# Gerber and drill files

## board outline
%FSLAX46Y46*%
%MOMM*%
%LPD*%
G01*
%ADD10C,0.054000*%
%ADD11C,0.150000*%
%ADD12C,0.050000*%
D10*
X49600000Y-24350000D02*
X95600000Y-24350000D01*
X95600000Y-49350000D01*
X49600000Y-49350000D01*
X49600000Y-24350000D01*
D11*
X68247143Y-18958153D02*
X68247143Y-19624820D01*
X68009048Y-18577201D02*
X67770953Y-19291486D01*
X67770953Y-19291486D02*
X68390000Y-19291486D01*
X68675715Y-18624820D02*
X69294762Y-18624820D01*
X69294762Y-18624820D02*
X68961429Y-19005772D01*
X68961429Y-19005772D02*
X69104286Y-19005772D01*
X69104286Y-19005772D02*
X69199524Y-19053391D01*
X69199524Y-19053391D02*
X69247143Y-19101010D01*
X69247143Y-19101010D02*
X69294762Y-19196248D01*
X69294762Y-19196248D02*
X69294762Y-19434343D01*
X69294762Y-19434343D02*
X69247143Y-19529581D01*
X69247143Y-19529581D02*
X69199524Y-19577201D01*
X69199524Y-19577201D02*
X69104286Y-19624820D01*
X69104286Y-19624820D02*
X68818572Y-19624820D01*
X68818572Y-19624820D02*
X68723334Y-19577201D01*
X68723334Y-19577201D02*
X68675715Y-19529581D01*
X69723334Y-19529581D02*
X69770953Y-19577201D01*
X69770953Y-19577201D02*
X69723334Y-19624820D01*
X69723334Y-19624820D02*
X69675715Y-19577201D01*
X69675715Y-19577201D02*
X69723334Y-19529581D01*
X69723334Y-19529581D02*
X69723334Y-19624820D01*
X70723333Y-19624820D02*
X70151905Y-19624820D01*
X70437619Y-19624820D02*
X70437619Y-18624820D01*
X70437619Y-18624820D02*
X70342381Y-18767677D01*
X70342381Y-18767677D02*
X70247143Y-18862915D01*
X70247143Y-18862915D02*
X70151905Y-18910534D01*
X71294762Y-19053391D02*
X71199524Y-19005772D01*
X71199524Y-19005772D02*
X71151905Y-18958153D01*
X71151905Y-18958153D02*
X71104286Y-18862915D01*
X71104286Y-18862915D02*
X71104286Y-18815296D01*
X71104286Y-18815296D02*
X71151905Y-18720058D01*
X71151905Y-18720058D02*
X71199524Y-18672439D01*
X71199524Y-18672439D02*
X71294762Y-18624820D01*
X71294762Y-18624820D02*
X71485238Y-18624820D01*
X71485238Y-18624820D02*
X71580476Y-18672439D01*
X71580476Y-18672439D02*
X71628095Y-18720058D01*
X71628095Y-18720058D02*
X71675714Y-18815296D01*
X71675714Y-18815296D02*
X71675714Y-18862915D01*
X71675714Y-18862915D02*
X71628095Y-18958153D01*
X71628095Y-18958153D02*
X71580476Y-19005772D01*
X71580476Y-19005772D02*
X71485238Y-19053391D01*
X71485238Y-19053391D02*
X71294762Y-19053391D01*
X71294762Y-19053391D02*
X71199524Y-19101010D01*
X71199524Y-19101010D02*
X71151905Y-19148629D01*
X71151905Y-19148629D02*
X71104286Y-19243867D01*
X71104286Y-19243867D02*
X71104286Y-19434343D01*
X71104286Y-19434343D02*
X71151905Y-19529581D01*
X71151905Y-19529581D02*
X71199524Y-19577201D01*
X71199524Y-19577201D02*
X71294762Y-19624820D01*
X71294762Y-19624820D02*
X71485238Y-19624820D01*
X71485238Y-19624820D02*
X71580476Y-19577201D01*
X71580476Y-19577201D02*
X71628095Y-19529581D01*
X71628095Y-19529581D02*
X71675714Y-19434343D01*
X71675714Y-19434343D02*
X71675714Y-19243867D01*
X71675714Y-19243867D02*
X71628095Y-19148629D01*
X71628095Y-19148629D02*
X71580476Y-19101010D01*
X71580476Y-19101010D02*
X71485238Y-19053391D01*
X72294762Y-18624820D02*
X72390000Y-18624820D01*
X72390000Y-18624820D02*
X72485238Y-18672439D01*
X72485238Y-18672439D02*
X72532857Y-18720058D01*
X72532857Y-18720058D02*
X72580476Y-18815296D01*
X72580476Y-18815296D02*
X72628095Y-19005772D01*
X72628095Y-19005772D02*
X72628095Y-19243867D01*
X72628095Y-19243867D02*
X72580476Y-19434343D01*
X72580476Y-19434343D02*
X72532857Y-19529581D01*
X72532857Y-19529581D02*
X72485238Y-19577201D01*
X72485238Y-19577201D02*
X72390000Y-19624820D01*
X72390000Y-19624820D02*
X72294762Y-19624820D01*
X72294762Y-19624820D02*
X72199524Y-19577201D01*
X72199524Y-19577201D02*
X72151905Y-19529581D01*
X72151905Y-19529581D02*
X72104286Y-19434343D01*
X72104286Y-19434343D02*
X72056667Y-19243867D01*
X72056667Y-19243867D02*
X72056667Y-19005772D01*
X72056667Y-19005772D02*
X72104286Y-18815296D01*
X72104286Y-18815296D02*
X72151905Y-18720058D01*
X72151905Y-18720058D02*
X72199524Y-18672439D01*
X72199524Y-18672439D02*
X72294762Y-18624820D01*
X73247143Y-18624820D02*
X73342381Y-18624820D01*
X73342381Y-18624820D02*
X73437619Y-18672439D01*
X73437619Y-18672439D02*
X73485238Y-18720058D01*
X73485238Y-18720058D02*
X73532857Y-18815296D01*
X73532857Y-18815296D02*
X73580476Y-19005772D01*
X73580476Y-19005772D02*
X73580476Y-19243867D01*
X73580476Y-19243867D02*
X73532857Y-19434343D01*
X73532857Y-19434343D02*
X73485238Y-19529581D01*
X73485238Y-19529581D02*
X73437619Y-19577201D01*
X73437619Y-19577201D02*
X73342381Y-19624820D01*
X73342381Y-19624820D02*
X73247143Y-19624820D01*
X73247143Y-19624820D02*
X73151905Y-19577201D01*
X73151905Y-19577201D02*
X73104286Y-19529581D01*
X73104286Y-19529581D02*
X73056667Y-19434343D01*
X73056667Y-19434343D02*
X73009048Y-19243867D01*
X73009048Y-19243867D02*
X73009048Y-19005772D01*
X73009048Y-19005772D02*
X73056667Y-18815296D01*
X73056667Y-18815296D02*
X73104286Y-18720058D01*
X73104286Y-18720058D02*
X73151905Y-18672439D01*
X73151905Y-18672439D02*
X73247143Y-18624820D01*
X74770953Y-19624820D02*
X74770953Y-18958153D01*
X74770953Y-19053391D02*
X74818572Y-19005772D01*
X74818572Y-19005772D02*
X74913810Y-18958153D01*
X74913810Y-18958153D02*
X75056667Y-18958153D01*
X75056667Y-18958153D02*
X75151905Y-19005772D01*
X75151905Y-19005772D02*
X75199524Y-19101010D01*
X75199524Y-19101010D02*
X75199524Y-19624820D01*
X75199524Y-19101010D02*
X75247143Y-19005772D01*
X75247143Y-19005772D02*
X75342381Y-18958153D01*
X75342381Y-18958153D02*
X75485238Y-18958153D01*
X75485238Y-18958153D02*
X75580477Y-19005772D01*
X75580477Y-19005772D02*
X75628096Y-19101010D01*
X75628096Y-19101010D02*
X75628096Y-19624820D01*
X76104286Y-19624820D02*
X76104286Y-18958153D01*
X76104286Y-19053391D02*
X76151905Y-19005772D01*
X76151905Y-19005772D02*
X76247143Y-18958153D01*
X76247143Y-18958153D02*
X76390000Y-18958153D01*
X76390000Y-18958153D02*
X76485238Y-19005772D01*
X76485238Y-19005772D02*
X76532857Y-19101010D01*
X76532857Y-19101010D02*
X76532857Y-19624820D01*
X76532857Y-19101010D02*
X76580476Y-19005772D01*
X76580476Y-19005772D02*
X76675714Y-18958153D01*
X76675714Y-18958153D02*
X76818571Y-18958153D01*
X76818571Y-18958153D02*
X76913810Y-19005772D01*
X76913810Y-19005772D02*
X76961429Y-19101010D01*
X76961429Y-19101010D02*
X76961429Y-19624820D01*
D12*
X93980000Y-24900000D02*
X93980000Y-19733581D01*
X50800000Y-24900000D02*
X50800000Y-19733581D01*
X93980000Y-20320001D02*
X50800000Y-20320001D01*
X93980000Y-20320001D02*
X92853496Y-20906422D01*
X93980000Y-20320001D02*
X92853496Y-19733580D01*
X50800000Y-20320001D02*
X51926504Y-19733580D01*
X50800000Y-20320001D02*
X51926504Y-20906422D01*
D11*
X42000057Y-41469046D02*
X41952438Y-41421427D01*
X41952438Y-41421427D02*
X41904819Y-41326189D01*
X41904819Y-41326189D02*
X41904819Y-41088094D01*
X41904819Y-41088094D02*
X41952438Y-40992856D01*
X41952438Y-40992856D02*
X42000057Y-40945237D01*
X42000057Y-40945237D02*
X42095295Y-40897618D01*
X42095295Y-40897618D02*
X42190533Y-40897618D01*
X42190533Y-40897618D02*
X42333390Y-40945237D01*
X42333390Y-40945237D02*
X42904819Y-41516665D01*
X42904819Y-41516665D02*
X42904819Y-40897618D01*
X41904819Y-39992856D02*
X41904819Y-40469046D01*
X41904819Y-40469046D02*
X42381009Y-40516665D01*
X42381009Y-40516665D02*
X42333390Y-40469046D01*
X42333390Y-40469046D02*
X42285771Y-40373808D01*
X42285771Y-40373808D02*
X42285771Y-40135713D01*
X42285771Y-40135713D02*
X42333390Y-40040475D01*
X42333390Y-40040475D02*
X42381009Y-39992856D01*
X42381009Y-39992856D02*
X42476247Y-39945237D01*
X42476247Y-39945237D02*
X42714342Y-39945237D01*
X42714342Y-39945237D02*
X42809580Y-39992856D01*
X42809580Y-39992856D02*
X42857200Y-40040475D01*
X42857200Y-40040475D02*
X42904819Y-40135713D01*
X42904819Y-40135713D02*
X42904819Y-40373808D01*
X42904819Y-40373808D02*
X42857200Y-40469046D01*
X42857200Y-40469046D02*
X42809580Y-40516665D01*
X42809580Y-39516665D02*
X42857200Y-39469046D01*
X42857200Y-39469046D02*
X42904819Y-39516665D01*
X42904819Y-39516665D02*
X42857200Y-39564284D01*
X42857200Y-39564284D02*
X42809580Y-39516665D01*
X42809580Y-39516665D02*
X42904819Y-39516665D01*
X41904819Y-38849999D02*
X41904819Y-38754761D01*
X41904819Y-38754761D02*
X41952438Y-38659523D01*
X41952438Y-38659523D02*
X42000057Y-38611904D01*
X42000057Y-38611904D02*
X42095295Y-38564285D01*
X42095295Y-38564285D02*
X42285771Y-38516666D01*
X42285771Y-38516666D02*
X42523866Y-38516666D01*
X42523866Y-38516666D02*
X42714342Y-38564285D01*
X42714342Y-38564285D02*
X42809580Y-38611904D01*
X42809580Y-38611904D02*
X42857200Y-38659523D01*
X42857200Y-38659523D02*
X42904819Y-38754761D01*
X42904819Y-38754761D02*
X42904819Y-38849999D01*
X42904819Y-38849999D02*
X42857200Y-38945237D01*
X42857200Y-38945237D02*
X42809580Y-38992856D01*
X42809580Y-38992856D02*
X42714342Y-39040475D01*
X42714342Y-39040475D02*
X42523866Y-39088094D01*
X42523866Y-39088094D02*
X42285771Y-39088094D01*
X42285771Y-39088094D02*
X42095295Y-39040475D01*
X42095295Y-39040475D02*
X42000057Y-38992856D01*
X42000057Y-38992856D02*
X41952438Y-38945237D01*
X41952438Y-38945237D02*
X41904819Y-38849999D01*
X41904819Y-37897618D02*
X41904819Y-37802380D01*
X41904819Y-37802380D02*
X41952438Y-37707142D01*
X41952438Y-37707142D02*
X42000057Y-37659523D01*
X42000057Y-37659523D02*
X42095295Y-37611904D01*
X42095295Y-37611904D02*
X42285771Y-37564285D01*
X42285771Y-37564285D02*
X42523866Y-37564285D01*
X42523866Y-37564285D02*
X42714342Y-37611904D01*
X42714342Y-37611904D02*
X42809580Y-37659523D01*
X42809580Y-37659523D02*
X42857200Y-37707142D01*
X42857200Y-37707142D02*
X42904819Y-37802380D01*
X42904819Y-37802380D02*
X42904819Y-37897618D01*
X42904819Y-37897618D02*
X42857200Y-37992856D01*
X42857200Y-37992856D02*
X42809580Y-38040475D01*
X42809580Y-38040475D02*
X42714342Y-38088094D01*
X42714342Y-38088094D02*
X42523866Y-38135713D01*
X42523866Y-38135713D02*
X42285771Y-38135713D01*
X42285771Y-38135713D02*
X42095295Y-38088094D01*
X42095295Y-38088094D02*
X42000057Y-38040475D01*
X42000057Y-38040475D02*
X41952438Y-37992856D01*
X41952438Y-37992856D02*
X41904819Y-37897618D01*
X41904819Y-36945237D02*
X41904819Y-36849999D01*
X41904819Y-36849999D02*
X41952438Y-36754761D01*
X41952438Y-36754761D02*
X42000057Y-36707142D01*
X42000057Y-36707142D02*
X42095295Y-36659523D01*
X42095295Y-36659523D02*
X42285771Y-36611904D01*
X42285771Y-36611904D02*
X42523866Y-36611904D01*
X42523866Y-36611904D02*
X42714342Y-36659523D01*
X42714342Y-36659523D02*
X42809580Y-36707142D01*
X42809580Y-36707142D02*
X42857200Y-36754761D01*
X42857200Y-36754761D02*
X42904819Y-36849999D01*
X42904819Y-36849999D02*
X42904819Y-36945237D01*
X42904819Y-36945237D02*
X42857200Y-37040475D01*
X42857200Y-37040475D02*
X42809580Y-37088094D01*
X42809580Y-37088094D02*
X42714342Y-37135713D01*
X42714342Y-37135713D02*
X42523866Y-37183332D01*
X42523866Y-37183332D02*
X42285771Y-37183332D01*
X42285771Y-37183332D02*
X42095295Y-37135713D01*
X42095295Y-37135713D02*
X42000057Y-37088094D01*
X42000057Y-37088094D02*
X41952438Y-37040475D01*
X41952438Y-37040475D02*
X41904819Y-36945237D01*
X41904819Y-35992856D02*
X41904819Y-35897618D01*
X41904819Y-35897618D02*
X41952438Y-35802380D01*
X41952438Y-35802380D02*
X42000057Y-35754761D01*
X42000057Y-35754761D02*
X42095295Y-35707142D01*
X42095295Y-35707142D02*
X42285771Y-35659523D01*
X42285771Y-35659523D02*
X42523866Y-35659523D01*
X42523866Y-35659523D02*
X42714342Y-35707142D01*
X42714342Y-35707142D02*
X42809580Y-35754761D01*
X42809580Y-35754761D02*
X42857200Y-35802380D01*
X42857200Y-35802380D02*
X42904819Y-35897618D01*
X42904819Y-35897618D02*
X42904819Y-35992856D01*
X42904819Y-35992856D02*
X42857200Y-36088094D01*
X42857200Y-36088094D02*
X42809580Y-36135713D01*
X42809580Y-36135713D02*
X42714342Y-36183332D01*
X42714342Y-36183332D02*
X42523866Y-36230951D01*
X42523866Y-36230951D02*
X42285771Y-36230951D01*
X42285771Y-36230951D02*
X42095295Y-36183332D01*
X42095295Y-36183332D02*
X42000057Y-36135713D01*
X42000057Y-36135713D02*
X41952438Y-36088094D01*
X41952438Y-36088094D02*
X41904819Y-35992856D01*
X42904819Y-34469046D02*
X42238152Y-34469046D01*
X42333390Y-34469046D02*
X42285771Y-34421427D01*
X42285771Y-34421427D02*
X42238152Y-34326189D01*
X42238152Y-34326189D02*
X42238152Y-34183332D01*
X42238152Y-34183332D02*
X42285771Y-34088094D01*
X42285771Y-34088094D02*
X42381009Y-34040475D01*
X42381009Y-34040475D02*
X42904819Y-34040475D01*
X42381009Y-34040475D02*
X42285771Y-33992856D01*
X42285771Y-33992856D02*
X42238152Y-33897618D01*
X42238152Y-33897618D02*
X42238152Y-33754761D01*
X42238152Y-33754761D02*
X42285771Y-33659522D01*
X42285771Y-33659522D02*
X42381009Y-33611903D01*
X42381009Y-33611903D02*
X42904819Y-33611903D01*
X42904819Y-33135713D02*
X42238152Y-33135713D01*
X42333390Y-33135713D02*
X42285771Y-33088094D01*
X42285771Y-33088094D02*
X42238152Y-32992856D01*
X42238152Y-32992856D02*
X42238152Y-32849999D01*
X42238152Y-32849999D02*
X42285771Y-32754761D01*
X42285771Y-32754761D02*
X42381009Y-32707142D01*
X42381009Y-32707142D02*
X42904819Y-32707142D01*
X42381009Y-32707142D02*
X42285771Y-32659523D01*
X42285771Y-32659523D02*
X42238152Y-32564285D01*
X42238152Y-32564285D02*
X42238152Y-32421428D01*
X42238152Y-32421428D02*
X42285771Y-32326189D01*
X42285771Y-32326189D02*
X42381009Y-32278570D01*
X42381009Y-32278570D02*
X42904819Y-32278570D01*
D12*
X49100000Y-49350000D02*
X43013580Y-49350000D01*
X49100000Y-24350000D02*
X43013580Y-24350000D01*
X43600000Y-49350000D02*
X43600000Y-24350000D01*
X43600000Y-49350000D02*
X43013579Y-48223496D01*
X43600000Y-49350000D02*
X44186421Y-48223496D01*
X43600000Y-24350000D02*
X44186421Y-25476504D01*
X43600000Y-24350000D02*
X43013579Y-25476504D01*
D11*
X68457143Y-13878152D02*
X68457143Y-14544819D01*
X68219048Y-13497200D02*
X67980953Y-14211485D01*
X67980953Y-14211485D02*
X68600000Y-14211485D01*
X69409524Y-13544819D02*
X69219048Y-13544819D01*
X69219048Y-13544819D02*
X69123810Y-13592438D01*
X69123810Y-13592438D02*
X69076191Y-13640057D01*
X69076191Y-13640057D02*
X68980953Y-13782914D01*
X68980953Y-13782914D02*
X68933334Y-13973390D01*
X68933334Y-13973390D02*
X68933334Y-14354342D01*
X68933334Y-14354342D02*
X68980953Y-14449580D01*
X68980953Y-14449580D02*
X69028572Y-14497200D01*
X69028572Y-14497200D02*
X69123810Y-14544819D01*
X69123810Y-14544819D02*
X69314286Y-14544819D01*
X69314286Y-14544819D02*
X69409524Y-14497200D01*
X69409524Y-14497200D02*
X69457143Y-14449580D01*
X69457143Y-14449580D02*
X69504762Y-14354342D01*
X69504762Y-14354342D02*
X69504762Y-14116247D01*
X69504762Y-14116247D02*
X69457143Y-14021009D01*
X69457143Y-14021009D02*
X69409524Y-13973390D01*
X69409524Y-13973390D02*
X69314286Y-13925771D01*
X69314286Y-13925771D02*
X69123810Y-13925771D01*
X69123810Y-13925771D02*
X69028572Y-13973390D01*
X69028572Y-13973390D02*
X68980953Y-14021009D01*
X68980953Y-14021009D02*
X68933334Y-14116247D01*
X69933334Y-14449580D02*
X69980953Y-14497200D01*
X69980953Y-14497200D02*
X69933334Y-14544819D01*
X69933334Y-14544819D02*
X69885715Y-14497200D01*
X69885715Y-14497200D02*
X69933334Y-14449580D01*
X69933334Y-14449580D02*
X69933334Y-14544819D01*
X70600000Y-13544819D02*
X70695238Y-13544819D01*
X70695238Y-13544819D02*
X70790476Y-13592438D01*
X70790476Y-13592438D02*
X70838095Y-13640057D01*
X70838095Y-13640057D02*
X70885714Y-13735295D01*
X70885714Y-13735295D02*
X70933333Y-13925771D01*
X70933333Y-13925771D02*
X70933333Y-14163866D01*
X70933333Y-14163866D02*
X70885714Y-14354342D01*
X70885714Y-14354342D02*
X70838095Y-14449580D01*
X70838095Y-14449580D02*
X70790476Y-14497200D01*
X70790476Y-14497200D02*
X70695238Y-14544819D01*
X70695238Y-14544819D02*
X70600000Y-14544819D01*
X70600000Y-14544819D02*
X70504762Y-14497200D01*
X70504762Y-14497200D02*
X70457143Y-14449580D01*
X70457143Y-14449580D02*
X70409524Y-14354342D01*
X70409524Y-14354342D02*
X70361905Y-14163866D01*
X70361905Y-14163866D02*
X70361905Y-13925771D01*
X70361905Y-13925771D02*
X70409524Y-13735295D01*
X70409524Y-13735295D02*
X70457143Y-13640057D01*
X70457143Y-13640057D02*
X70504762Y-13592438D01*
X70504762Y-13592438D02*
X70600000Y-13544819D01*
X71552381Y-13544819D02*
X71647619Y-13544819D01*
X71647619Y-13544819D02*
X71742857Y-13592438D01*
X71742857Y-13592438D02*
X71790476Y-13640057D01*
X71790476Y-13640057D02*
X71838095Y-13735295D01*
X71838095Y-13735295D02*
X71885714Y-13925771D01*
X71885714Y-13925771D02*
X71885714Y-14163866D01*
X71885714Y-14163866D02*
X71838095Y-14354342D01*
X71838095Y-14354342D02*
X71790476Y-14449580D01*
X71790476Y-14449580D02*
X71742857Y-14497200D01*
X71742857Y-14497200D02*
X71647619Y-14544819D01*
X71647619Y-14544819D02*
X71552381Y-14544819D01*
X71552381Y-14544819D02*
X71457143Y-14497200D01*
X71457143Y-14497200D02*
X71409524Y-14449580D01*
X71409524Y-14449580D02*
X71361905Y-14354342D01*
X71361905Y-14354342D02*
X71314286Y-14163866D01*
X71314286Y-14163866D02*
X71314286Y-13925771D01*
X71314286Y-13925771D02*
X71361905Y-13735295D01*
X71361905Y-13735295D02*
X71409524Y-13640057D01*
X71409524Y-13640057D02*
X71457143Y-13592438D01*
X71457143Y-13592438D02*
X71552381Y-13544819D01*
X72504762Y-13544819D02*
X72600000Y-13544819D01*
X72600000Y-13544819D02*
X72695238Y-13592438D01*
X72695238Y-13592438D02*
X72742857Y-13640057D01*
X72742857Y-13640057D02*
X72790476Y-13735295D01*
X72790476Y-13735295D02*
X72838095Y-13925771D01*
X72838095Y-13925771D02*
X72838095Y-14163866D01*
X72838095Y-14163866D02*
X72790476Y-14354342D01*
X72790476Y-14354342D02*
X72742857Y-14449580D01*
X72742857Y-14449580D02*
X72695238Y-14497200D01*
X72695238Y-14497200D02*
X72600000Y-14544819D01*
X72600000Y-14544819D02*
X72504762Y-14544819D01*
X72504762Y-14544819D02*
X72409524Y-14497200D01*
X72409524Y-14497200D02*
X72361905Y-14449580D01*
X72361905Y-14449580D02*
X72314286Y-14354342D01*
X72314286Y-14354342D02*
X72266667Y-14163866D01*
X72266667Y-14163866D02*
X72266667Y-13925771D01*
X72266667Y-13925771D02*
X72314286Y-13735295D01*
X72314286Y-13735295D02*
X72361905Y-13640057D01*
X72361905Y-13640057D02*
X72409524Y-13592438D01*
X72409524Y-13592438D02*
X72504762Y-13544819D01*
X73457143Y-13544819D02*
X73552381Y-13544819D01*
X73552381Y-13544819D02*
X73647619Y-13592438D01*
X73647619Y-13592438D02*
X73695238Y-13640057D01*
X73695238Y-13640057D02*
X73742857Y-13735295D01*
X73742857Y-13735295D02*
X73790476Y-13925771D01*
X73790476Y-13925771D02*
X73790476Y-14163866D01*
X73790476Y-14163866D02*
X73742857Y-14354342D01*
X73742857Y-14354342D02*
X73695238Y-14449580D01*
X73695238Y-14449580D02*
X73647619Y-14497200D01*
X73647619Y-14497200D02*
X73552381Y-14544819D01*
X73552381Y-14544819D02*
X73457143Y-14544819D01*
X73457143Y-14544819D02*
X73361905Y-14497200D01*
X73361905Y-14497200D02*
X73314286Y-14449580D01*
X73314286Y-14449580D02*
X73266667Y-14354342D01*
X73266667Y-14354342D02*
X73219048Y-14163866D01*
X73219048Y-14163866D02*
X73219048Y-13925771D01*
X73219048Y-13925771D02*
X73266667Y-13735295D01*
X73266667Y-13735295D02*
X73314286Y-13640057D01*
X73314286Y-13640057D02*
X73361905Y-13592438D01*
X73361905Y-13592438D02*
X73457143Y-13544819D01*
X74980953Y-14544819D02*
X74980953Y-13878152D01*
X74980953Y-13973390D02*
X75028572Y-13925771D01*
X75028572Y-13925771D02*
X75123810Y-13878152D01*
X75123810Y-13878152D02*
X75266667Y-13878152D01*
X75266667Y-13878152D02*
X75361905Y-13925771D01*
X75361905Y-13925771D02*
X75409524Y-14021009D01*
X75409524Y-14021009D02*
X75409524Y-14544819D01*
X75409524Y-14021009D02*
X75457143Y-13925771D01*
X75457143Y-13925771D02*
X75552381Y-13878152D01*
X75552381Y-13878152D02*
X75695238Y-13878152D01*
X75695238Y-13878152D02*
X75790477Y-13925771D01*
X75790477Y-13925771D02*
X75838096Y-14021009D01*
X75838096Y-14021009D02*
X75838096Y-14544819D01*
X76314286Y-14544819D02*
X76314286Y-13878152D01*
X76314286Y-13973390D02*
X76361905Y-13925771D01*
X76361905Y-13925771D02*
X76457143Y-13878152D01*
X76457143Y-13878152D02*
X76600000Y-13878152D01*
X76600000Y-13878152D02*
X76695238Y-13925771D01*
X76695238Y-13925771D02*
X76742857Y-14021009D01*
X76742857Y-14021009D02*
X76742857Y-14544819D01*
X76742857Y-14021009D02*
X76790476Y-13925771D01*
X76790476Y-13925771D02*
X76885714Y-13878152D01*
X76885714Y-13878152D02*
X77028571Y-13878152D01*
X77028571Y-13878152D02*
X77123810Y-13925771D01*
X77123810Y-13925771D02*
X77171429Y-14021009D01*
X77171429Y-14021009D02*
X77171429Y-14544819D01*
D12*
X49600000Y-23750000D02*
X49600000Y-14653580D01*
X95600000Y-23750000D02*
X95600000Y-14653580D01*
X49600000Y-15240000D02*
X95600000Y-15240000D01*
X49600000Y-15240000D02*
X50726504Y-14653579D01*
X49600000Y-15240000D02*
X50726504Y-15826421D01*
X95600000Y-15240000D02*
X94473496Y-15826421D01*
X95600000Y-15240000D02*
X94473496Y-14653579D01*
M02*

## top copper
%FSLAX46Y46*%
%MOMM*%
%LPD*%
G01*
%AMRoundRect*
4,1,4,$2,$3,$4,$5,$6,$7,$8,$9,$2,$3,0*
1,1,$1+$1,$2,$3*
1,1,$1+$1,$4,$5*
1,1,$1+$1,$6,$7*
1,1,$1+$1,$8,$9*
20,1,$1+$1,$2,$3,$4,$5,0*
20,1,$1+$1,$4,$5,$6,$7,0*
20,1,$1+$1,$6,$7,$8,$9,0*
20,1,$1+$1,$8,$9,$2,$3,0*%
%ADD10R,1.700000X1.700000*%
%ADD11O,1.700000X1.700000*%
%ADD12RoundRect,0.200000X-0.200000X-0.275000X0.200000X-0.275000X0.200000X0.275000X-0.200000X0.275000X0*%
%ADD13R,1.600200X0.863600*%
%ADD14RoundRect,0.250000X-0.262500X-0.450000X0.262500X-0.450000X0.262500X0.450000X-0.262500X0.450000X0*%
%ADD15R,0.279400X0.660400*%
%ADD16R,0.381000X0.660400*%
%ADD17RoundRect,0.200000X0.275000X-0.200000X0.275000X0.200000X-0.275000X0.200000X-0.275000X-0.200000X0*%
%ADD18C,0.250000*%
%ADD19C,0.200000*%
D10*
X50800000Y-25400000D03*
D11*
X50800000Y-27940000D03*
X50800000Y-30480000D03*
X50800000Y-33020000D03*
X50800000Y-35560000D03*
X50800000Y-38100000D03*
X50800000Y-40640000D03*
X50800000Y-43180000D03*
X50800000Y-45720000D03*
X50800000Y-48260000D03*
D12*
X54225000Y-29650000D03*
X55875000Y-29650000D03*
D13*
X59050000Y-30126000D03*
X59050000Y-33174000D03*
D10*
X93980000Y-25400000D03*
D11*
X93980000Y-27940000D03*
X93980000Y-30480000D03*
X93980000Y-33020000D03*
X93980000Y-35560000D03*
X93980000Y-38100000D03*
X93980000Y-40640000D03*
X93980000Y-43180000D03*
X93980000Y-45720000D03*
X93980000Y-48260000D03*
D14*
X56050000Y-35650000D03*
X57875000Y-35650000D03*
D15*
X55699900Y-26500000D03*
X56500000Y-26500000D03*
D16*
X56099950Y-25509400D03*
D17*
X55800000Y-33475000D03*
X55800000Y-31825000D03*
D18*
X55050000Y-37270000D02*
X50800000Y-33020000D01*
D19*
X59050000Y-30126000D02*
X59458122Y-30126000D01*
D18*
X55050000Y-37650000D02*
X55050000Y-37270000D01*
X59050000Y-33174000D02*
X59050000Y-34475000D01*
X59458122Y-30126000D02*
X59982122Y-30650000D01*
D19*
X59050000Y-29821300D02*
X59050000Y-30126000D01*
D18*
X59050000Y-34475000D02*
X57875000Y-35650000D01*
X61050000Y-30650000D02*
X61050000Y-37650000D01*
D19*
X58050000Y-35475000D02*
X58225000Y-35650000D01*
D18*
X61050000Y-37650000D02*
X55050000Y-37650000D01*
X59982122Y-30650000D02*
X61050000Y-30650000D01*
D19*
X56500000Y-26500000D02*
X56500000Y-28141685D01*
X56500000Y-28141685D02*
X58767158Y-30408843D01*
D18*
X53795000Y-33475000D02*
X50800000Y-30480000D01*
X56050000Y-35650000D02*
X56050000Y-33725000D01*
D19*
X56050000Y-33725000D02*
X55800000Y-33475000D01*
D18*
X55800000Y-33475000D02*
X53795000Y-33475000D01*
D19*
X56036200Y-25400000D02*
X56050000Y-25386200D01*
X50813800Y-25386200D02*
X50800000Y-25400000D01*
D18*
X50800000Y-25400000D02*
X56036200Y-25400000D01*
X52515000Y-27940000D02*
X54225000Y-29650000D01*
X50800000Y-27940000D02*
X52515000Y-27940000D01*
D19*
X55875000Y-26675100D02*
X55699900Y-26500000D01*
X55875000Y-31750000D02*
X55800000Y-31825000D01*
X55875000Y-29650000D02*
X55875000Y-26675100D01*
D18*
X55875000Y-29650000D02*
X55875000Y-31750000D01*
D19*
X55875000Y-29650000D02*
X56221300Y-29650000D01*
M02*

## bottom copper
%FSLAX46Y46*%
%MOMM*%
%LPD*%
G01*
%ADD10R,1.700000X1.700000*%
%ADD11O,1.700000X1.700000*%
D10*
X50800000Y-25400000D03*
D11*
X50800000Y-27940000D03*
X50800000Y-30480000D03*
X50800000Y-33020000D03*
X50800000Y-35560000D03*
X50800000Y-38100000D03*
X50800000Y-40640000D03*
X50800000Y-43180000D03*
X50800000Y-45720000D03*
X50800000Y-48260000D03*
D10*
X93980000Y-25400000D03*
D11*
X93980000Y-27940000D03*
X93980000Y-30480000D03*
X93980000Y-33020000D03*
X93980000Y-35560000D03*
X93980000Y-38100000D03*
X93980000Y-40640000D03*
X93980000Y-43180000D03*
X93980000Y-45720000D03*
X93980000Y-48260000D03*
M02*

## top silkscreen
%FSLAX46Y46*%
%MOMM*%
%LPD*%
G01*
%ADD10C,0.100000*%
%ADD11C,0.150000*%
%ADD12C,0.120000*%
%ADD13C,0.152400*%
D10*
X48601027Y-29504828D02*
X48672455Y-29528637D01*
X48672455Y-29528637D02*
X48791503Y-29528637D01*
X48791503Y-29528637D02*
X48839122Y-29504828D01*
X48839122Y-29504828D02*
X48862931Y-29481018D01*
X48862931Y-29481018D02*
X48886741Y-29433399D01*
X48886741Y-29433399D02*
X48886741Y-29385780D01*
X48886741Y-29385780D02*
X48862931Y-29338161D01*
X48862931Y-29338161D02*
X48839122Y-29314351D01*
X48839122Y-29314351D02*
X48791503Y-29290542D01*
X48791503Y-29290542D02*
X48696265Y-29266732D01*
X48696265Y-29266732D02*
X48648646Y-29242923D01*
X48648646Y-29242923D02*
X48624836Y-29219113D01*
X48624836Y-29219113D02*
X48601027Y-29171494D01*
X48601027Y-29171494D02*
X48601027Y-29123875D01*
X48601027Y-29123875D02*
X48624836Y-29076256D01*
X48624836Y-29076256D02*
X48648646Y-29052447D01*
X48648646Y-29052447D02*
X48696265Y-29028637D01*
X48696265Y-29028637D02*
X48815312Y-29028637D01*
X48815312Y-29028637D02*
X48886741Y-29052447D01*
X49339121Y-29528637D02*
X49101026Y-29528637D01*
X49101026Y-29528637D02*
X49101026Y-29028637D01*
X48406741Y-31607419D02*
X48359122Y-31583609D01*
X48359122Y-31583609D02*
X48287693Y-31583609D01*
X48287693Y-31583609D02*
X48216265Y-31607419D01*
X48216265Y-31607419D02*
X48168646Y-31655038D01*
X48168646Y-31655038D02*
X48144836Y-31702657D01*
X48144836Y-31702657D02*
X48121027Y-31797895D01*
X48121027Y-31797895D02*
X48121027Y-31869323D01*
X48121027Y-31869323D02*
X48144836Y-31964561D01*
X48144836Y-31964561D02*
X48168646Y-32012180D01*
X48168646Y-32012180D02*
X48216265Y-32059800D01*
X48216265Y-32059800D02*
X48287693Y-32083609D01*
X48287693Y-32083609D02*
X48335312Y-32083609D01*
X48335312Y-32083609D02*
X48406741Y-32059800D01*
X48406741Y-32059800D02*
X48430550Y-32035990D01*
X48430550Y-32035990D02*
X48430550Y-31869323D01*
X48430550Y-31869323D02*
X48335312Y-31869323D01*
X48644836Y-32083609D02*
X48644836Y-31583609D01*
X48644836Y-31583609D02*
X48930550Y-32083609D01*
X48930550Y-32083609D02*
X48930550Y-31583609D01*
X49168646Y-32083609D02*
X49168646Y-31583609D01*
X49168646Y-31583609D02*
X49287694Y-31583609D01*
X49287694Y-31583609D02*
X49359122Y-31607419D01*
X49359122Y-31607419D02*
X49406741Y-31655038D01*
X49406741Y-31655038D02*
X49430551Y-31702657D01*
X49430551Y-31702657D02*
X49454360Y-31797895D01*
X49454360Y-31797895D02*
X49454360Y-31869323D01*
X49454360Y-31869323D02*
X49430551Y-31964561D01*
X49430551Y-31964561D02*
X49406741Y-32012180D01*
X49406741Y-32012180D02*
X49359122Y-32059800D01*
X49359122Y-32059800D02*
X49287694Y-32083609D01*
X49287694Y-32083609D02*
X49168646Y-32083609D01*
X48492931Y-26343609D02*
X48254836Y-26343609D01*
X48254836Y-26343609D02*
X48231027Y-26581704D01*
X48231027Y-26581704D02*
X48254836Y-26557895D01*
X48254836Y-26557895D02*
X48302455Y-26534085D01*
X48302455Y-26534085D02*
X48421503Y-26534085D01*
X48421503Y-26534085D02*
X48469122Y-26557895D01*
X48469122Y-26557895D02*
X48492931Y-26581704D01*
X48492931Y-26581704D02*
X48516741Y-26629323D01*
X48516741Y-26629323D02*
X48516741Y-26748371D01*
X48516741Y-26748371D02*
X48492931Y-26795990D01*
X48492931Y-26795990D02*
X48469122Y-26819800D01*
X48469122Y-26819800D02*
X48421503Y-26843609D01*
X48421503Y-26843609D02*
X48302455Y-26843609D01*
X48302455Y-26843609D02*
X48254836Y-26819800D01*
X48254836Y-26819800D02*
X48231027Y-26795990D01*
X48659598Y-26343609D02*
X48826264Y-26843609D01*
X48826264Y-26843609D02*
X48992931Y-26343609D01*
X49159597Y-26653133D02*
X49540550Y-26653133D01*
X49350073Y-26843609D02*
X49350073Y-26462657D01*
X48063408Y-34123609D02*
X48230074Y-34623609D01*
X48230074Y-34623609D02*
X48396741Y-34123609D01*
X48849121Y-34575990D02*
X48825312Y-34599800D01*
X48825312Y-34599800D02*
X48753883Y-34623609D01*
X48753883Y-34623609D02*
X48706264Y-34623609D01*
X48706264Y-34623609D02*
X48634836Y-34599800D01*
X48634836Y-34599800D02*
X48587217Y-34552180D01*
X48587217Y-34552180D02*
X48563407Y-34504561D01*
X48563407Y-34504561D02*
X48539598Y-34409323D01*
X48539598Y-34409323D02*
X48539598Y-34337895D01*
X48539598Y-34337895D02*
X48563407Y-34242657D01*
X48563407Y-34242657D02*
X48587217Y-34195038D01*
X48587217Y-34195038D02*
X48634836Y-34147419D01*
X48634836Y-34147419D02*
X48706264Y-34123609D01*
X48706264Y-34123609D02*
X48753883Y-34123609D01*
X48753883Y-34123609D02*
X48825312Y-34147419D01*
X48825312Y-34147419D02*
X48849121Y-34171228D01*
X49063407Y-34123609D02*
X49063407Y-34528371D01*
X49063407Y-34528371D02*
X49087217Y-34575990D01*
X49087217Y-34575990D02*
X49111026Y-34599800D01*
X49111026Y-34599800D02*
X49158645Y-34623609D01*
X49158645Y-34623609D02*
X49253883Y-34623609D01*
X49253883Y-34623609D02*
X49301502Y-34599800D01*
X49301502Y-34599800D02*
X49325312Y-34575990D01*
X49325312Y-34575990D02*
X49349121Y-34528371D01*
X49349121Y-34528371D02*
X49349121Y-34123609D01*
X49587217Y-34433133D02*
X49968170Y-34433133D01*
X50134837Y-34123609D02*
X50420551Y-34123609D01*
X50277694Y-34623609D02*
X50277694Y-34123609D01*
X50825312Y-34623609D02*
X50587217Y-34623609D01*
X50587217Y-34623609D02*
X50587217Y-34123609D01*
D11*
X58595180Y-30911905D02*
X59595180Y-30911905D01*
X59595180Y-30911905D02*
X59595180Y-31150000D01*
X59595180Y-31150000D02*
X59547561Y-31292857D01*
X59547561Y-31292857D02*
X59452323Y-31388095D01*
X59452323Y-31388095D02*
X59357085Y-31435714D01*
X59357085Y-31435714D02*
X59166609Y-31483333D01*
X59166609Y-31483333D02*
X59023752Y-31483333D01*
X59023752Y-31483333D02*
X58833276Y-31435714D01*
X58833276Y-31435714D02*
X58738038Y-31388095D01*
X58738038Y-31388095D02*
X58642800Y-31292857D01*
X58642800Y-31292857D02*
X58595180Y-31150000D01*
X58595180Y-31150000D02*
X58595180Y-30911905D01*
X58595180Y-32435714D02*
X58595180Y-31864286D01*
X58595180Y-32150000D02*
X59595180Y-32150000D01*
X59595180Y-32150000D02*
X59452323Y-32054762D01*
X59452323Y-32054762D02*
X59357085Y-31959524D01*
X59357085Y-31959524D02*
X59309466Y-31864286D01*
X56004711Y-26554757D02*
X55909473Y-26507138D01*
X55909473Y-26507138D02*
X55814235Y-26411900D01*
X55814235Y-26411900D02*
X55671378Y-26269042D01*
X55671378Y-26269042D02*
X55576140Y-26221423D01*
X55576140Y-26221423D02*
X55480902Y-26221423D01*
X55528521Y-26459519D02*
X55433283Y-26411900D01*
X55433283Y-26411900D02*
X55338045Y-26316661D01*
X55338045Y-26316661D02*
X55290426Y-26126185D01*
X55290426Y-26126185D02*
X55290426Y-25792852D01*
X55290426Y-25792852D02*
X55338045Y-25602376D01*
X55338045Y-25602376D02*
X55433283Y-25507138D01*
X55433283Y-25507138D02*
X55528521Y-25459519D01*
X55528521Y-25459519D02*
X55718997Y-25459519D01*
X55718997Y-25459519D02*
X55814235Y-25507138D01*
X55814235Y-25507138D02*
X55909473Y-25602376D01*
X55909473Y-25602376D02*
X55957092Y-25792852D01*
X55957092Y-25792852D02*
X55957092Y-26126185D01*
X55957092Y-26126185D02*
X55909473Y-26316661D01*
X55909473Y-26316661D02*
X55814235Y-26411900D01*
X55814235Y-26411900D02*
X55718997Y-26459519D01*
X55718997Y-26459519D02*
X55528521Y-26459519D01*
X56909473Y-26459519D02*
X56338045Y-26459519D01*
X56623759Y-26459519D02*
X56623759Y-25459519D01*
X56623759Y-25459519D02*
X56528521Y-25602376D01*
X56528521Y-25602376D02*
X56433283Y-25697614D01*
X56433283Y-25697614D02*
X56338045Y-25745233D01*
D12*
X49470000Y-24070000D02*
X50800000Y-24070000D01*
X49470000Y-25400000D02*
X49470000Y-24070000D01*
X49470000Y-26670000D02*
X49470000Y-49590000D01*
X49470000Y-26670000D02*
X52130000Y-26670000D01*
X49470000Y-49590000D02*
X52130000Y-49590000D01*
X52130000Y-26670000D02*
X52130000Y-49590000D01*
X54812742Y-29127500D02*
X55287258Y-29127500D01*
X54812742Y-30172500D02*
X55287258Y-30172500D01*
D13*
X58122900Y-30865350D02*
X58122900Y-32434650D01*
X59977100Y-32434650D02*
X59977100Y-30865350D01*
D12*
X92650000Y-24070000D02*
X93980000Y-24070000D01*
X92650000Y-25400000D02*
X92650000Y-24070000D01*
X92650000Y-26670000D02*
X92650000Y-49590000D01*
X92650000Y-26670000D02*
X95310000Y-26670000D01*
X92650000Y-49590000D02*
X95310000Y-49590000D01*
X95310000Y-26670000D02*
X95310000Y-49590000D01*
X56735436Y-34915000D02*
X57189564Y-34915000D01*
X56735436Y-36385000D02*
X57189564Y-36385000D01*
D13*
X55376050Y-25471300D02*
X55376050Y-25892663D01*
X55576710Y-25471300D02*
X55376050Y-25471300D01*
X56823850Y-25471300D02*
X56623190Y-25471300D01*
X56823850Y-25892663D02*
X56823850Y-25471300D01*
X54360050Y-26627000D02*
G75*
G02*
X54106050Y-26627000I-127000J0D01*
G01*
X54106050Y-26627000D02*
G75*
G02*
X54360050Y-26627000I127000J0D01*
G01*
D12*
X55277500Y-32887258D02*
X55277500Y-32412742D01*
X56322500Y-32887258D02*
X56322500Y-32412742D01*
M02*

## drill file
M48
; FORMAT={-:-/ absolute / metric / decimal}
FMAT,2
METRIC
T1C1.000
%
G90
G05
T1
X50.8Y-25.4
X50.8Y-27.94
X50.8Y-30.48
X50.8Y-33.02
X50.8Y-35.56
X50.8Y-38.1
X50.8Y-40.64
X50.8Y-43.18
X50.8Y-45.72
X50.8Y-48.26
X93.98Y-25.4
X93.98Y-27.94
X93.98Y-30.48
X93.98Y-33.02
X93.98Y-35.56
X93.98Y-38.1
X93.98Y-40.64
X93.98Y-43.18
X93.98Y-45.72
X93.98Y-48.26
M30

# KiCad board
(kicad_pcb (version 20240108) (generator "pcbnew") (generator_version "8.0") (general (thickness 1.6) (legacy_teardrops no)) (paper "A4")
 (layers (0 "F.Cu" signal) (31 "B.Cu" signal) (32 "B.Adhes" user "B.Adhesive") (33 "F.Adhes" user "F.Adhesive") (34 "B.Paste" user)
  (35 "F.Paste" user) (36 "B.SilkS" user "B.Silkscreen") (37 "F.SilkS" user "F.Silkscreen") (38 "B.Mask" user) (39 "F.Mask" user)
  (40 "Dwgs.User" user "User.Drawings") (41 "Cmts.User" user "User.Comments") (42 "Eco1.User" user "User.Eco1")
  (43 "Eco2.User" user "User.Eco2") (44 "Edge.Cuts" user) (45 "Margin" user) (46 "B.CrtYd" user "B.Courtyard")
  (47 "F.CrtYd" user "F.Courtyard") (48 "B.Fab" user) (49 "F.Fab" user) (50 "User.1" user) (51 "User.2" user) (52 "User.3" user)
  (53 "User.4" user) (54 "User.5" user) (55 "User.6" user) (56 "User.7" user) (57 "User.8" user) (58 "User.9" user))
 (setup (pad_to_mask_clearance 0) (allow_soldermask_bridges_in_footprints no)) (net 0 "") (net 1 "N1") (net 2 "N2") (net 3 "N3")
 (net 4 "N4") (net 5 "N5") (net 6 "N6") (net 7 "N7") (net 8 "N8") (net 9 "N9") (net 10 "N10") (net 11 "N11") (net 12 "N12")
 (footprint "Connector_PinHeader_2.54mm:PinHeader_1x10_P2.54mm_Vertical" (layer "F.Cu") (at 50.8 25.4)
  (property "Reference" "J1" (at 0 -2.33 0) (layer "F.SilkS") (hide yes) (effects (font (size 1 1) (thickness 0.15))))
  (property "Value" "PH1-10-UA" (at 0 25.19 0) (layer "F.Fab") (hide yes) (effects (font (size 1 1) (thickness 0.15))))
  (fp_line (start -1.33 -1.33) (end 0 -1.33) (stroke (width 0.12) (type solid)) (layer "F.SilkS"))
  (fp_line (start -1.33 0) (end -1.33 -1.33) (stroke (width 0.12) (type solid)) (layer "F.SilkS"))
  (fp_line (start -1.33 1.27) (end -1.33 24.19) (stroke (width 0.12) (type solid)) (layer "F.SilkS"))
  (fp_line (start -1.33 1.27) (end 1.33 1.27) (stroke (width 0.12) (type solid)) (layer "F.SilkS"))
  (fp_line (start -1.33 24.19) (end 1.33 24.19) (stroke (width 0.12) (type solid)) (layer "F.SilkS"))
  (fp_line (start 1.33 1.27) (end 1.33 24.19) (stroke (width 0.12) (type solid)) (layer "F.SilkS"))
  (pad "1" thru_hole rect (at 0 0) (size 1.7 1.7) (drill 1) (layers "*.Cu" "*.Mask") (remove_unused_layers no) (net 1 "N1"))
  (pad "2" thru_hole oval (at 0 2.54) (size 1.7 1.7) (drill 1) (layers "*.Cu" "*.Mask") (remove_unused_layers no) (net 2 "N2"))
  (pad "3" thru_hole oval (at 0 5.08) (size 1.7 1.7) (drill 1) (layers "*.Cu" "*.Mask") (remove_unused_layers no) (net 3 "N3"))
  (pad "4" thru_hole oval (at 0 7.62) (size 1.7 1.7) (drill 1) (layers "*.Cu" "*.Mask") (remove_unused_layers no) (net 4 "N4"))
  (pad "5" thru_hole oval (at 0 10.16) (size 1.7 1.7) (drill 1) (layers "*.Cu" "*.Mask") (remove_unused_layers no) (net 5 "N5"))
  (pad "6" thru_hole oval (at 0 12.7) (size 1.7 1.7) (drill 1) (layers "*.Cu" "*.Mask") (remove_unused_layers no) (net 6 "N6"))
  (pad "7" thru_hole oval (at 0 15.24) (size 1.7 1.7) (drill 1) (layers "*.Cu" "*.Mask") (remove_unused_layers no) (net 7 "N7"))
  (pad "8" thru_hole oval (at 0 17.78) (size 1.7 1.7) (drill 1) (layers "*.Cu" "*.Mask") (remove_unused_layers no) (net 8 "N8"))
  (pad "9" thru_hole oval (at 0 20.32) (size 1.7 1.7) (drill 1) (layers "*.Cu" "*.Mask") (remove_unused_layers no) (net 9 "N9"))
  (pad "10" thru_hole oval (at 0 22.86) (size 1.7 1.7) (drill 1) (layers "*.Cu" "*.Mask") (remove_unused_layers no) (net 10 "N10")))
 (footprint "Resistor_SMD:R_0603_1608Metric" (layer "F.Cu") (at 55.05 29.65)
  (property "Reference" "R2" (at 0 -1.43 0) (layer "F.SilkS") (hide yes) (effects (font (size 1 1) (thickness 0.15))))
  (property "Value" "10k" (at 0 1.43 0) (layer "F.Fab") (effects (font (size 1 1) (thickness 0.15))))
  (fp_line (start -0.237258 -0.5225) (end 0.237258 -0.5225) (stroke (width 0.12) (type solid)) (layer "F.SilkS"))
  (fp_line (start -0.237258 0.5225) (end 0.237258 0.5225) (stroke (width 0.12) (type solid)) (layer "F.SilkS"))
  (pad "1" smd roundrect (at -0.825 0) (size 0.8 0.95) (layers "F.Cu" "F.Paste" "F.Mask") (roundrect_rratio 0.25) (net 2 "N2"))
  (pad "2" smd roundrect (at 0.825 0) (size 0.8 0.95) (layers "F.Cu" "F.Paste" "F.Mask") (roundrect_rratio 0.25) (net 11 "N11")))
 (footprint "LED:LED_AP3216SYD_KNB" (layer "F.Cu") (at 59.05 31.65 -90)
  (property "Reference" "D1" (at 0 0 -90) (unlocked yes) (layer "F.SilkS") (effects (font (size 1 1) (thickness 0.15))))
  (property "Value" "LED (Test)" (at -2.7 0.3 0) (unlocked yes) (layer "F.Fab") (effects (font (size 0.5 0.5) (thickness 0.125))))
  (fp_line (start -0.78465 0.9271) (end 0.78465 0.9271) (stroke (width 0.1524) (type solid)) (layer "F.SilkS"))
  (fp_line (start 0.78465 -0.9271) (end -0.78465 -0.9271) (stroke (width 0.1524) (type solid)) (layer "F.SilkS"))
  (pad "1" smd rect (at -1.524 0 270) (size 0.8636 1.6002) (layers "F.Cu" "F.Paste" "F.Mask") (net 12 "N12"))
  (pad "2" smd rect (at 1.524 0 270) (size 0.8636 1.6002) (layers "F.Cu" "F.Paste" "F.Mask") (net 4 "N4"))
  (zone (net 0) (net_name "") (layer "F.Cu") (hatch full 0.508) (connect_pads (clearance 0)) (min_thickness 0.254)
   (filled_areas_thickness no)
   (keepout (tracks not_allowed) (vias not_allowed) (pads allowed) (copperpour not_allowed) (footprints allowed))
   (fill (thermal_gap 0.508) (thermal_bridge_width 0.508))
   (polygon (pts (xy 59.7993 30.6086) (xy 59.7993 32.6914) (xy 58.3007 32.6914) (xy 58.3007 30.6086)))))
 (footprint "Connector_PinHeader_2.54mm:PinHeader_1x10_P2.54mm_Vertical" (layer "F.Cu") (at 93.98 25.4)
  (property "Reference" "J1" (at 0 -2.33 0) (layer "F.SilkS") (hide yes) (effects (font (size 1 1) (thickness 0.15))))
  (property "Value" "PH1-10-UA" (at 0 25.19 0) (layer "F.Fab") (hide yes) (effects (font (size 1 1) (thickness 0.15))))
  (fp_line (start -1.33 -1.33) (end 0 -1.33) (stroke (width 0.12) (type solid)) (layer "F.SilkS"))
  (fp_line (start -1.33 0) (end -1.33 -1.33) (stroke (width 0.12) (type solid)) (layer "F.SilkS"))
  (fp_line (start -1.33 1.27) (end -1.33 24.19) (stroke (width 0.12) (type solid)) (layer "F.SilkS"))
  (fp_line (start -1.33 1.27) (end 1.33 1.27) (stroke (width 0.12) (type solid)) (layer "F.SilkS"))
  (fp_line (start -1.33 24.19) (end 1.33 24.19) (stroke (width 0.12) (type solid)) (layer "F.SilkS"))
  (fp_line (start 1.33 1.27) (end 1.33 24.19) (stroke (width 0.12) (type solid)) (layer "F.SilkS"))
  (pad "1" thru_hole rect (at 0 0) (size 1.7 1.7) (drill 1) (layers "*.Cu" "*.Mask") (remove_unused_layers no))
  (pad "2" thru_hole oval (at 0 2.54) (size 1.7 1.7) (drill 1) (layers "*.Cu" "*.Mask") (remove_unused_layers no))
  (pad "3" thru_hole oval (at 0 5.08) (size 1.7 1.7) (drill 1) (layers "*.Cu" "*.Mask") (remove_unused_layers no))
  (pad "4" thru_hole oval (at 0 7.62) (size 1.7 1.7) (drill 1) (layers "*.Cu" "*.Mask") (remove_unused_layers no))
  (pad "5" thru_hole oval (at 0 10.16) (size 1.7 1.7) (drill 1) (layers "*.Cu" "*.Mask") (remove_unused_layers no))
  (pad "6" thru_hole oval (at 0 12.7) (size 1.7 1.7) (drill 1) (layers "*.Cu" "*.Mask") (remove_unused_layers no))
  (pad "7" thru_hole oval (at 0 15.24) (size 1.7 1.7) (drill 1) (layers "*.Cu" "*.Mask") (remove_unused_layers no))
  (pad "8" thru_hole oval (at 0 17.78) (size 1.7 1.7) (drill 1) (layers "*.Cu" "*.Mask") (remove_unused_layers no))
  (pad "9" thru_hole oval (at 0 20.32) (size 1.7 1.7) (drill 1) (layers "*.Cu" "*.Mask") (remove_unused_layers no))
  (pad "10" thru_hole oval (at 0 22.86) (size 1.7 1.7) (drill 1) (layers "*.Cu" "*.Mask") (remove_unused_layers no)))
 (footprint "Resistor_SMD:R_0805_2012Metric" (layer "F.Cu") (at 56.9625 35.65)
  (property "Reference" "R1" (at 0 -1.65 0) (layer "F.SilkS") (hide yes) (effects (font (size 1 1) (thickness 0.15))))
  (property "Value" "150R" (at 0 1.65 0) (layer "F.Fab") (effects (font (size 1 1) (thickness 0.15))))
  (fp_line (start -0.227064 -0.735) (end 0.227064 -0.735) (stroke (width 0.12) (type solid)) (layer "F.SilkS"))
  (fp_line (start -0.227064 0.735) (end 0.227064 0.735) (stroke (width 0.12) (type solid)) (layer "F.SilkS"))
  (pad "1" smd roundrect (at -0.9125 0) (size 1.025 1.4) (layers "F.Cu" "F.Paste" "F.Mask") (roundrect_rratio 0.243902) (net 3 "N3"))
  (pad "2" smd roundrect (at 0.9125 0) (size 1.025 1.4) (layers "F.Cu" "F.Paste" "F.Mask") (roundrect_rratio 0.243902) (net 12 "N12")))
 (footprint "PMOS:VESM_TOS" (layer "F.Cu") (at 56.09995 26.0047)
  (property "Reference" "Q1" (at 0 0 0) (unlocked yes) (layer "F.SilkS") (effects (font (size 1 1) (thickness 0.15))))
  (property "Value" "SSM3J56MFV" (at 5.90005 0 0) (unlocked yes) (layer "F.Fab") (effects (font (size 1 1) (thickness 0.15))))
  (fp_line (start -0.7239 -0.5334) (end -0.7239 -0.112037) (stroke (width 0.1524) (type solid)) (layer "F.SilkS"))
  (fp_line (start -0.52324 -0.5334) (end -0.7239 -0.5334) (stroke (width 0.1524) (type solid)) (layer "F.SilkS"))
  (fp_line (start 0.7239 -0.5334) (end 0.52324 -0.5334) (stroke (width 0.1524) (type solid)) (layer "F.SilkS"))
  (fp_line (start 0.7239 -0.112037) (end 0.7239 -0.5334) (stroke (width 0.1524) (type solid)) (layer "F.SilkS"))
  (fp_circle (center -1.8669 0.6223) (end -1.7399 0.6223) (stroke (width 0.1524) (type solid)) (fill none) (layer "F.SilkS"))
  (pad "1" smd rect (at -0.40005 0.4953) (size 0.2794 0.6604) (layers "F.Cu" "F.Paste" "F.Mask") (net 11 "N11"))
  (pad "2" smd rect (at 0.40005 0.4953) (size 0.2794 0.6604) (layers "F.Cu" "F.Paste" "F.Mask") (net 12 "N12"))
  (pad "3" smd rect (at 0 -0.4953) (size 0.381 0.6604) (layers "F.Cu" "F.Paste" "F.Mask") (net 1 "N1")))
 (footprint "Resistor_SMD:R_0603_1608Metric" (layer "F.Cu") (at 55.8 32.65 90)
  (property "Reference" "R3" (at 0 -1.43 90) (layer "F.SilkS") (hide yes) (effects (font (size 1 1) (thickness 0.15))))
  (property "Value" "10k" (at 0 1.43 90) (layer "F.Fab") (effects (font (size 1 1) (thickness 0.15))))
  (fp_line (start -0.237258 -0.5225) (end 0.237258 -0.5225) (stroke (width 0.12) (type solid)) (layer "F.SilkS"))
  (fp_line (start -0.237258 0.5225) (end 0.237258 0.5225) (stroke (width 0.12) (type solid)) (layer "F.SilkS"))
  (pad "1" smd roundrect (at -0.825 0 90) (size 0.8 0.95) (layers "F.Cu" "F.Paste" "F.Mask") (roundrect_rratio 0.25) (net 3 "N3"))
  (pad "2" smd roundrect (at 0.825 0 90) (size 0.8 0.95) (layers "F.Cu" "F.Paste" "F.Mask") (roundrect_rratio 0.25) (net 11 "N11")))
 (gr_rect (start 49.6 24.35) (end 95.6 49.35) (stroke (width 0.054) (type default)) (fill none) (layer "Edge.Cuts"))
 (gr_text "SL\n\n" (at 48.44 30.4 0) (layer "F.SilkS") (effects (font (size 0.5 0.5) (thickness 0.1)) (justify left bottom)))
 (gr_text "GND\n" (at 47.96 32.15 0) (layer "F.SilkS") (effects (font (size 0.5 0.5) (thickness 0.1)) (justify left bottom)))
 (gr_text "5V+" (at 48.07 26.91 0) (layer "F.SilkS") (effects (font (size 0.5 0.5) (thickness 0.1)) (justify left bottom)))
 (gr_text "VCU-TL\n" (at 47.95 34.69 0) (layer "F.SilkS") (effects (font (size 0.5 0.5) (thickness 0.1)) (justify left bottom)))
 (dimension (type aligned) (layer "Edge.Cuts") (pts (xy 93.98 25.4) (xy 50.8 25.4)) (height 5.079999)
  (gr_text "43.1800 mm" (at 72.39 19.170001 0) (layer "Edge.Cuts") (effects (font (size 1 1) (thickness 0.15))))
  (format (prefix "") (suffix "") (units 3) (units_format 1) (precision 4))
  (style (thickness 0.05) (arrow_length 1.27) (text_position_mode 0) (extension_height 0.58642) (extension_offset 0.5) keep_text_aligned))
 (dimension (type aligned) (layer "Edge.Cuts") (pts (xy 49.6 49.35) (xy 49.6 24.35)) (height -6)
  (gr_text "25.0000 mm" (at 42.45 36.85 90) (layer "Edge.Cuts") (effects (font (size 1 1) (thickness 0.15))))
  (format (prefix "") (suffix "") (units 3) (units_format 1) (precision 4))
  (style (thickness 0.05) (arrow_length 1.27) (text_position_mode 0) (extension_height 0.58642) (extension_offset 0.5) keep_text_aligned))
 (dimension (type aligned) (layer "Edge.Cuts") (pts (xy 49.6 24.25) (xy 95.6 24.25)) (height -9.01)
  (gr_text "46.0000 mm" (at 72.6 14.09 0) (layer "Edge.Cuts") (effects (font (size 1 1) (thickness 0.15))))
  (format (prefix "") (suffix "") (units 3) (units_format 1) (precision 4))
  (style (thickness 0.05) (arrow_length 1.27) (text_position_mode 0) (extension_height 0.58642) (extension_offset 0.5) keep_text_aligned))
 (segment (start 55.05 37.27) (end 50.8 33.02) (width 0.25) (layer "F.Cu") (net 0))
 (segment (start 59.05 30.126) (end 59.458122 30.126) (width 0.2) (layer "F.Cu") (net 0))
 (segment (start 55.05 37.65) (end 55.05 37.27) (width 0.25) (layer "F.Cu") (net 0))
 (segment (start 59.05 33.174) (end 59.05 34.475) (width 0.25) (layer "F.Cu") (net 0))
 (segment (start 59.458122 30.126) (end 59.982122 30.65) (width 0.25) (layer "F.Cu") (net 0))
 (segment (start 59.05 29.8213) (end 59.05 30.126) (width 0.2) (layer "F.Cu") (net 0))
 (segment (start 59.05 34.475) (end 57.875 35.65) (width 0.25) (layer "F.Cu") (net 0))
 (segment (start 61.05 30.65) (end 61.05 37.65) (width 0.25) (layer "F.Cu") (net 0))
 (segment (start 58.05 35.475) (end 58.225 35.65) (width 0.2) (layer "F.Cu") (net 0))
 (segment (start 61.05 37.65) (end 55.05 37.65) (width 0.25) (layer "F.Cu") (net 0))
 (segment (start 59.982122 30.65) (end 61.05 30.65) (width 0.25) (layer "F.Cu") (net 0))
 (segment (start 56.5 26.5) (end 56.5 28.141685) (width 0.2) (layer "F.Cu") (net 12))
 (segment (start 56.5 28.141685) (end 58.767158 30.408843) (width 0.2) (layer "F.Cu") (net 12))
 (segment (start 53.795 33.475) (end 50.8 30.48) (width 0.25) (layer "F.Cu") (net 3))
 (segment (start 56.05 35.65) (end 56.05 33.725) (width 0.25) (layer "F.Cu") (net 3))
 (segment (start 56.05 33.725) (end 55.8 33.475) (width 0.2) (layer "F.Cu") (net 3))
 (segment (start 55.8 33.475) (end 53.795 33.475) (width 0.25) (layer "F.Cu") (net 3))
 (segment (start 56.0362 25.4) (end 56.05 25.3862) (width 0.2) (layer "F.Cu") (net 1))
 (segment (start 50.8138 25.3862) (end 50.8 25.4) (width 0.2) (layer "F.Cu") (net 1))
 (segment (start 50.8 25.4) (end 56.0362 25.4) (width 0.25) (layer "F.Cu") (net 1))
 (segment (start 52.515 27.94) (end 54.225 29.65) (width 0.25) (layer "F.Cu") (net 2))
 (segment (start 50.8 27.94) (end 52.515 27.94) (width 0.25) (layer "F.Cu") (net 2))
 (segment (start 55.875 26.6751) (end 55.6999 26.5) (width 0.2) (layer "F.Cu") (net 11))
 (segment (start 55.875 31.75) (end 55.8 31.825) (width 0.2) (layer "F.Cu") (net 11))
 (segment (start 55.875 29.65) (end 55.875 26.6751) (width 0.2) (layer "F.Cu") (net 11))
 (segment (start 55.875 29.65) (end 55.875 31.75) (width 0.25) (layer "F.Cu") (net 11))
 (segment (start 55.875 29.65) (end 56.2213 29.65) (width 0.2) (layer "F.Cu") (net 11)))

